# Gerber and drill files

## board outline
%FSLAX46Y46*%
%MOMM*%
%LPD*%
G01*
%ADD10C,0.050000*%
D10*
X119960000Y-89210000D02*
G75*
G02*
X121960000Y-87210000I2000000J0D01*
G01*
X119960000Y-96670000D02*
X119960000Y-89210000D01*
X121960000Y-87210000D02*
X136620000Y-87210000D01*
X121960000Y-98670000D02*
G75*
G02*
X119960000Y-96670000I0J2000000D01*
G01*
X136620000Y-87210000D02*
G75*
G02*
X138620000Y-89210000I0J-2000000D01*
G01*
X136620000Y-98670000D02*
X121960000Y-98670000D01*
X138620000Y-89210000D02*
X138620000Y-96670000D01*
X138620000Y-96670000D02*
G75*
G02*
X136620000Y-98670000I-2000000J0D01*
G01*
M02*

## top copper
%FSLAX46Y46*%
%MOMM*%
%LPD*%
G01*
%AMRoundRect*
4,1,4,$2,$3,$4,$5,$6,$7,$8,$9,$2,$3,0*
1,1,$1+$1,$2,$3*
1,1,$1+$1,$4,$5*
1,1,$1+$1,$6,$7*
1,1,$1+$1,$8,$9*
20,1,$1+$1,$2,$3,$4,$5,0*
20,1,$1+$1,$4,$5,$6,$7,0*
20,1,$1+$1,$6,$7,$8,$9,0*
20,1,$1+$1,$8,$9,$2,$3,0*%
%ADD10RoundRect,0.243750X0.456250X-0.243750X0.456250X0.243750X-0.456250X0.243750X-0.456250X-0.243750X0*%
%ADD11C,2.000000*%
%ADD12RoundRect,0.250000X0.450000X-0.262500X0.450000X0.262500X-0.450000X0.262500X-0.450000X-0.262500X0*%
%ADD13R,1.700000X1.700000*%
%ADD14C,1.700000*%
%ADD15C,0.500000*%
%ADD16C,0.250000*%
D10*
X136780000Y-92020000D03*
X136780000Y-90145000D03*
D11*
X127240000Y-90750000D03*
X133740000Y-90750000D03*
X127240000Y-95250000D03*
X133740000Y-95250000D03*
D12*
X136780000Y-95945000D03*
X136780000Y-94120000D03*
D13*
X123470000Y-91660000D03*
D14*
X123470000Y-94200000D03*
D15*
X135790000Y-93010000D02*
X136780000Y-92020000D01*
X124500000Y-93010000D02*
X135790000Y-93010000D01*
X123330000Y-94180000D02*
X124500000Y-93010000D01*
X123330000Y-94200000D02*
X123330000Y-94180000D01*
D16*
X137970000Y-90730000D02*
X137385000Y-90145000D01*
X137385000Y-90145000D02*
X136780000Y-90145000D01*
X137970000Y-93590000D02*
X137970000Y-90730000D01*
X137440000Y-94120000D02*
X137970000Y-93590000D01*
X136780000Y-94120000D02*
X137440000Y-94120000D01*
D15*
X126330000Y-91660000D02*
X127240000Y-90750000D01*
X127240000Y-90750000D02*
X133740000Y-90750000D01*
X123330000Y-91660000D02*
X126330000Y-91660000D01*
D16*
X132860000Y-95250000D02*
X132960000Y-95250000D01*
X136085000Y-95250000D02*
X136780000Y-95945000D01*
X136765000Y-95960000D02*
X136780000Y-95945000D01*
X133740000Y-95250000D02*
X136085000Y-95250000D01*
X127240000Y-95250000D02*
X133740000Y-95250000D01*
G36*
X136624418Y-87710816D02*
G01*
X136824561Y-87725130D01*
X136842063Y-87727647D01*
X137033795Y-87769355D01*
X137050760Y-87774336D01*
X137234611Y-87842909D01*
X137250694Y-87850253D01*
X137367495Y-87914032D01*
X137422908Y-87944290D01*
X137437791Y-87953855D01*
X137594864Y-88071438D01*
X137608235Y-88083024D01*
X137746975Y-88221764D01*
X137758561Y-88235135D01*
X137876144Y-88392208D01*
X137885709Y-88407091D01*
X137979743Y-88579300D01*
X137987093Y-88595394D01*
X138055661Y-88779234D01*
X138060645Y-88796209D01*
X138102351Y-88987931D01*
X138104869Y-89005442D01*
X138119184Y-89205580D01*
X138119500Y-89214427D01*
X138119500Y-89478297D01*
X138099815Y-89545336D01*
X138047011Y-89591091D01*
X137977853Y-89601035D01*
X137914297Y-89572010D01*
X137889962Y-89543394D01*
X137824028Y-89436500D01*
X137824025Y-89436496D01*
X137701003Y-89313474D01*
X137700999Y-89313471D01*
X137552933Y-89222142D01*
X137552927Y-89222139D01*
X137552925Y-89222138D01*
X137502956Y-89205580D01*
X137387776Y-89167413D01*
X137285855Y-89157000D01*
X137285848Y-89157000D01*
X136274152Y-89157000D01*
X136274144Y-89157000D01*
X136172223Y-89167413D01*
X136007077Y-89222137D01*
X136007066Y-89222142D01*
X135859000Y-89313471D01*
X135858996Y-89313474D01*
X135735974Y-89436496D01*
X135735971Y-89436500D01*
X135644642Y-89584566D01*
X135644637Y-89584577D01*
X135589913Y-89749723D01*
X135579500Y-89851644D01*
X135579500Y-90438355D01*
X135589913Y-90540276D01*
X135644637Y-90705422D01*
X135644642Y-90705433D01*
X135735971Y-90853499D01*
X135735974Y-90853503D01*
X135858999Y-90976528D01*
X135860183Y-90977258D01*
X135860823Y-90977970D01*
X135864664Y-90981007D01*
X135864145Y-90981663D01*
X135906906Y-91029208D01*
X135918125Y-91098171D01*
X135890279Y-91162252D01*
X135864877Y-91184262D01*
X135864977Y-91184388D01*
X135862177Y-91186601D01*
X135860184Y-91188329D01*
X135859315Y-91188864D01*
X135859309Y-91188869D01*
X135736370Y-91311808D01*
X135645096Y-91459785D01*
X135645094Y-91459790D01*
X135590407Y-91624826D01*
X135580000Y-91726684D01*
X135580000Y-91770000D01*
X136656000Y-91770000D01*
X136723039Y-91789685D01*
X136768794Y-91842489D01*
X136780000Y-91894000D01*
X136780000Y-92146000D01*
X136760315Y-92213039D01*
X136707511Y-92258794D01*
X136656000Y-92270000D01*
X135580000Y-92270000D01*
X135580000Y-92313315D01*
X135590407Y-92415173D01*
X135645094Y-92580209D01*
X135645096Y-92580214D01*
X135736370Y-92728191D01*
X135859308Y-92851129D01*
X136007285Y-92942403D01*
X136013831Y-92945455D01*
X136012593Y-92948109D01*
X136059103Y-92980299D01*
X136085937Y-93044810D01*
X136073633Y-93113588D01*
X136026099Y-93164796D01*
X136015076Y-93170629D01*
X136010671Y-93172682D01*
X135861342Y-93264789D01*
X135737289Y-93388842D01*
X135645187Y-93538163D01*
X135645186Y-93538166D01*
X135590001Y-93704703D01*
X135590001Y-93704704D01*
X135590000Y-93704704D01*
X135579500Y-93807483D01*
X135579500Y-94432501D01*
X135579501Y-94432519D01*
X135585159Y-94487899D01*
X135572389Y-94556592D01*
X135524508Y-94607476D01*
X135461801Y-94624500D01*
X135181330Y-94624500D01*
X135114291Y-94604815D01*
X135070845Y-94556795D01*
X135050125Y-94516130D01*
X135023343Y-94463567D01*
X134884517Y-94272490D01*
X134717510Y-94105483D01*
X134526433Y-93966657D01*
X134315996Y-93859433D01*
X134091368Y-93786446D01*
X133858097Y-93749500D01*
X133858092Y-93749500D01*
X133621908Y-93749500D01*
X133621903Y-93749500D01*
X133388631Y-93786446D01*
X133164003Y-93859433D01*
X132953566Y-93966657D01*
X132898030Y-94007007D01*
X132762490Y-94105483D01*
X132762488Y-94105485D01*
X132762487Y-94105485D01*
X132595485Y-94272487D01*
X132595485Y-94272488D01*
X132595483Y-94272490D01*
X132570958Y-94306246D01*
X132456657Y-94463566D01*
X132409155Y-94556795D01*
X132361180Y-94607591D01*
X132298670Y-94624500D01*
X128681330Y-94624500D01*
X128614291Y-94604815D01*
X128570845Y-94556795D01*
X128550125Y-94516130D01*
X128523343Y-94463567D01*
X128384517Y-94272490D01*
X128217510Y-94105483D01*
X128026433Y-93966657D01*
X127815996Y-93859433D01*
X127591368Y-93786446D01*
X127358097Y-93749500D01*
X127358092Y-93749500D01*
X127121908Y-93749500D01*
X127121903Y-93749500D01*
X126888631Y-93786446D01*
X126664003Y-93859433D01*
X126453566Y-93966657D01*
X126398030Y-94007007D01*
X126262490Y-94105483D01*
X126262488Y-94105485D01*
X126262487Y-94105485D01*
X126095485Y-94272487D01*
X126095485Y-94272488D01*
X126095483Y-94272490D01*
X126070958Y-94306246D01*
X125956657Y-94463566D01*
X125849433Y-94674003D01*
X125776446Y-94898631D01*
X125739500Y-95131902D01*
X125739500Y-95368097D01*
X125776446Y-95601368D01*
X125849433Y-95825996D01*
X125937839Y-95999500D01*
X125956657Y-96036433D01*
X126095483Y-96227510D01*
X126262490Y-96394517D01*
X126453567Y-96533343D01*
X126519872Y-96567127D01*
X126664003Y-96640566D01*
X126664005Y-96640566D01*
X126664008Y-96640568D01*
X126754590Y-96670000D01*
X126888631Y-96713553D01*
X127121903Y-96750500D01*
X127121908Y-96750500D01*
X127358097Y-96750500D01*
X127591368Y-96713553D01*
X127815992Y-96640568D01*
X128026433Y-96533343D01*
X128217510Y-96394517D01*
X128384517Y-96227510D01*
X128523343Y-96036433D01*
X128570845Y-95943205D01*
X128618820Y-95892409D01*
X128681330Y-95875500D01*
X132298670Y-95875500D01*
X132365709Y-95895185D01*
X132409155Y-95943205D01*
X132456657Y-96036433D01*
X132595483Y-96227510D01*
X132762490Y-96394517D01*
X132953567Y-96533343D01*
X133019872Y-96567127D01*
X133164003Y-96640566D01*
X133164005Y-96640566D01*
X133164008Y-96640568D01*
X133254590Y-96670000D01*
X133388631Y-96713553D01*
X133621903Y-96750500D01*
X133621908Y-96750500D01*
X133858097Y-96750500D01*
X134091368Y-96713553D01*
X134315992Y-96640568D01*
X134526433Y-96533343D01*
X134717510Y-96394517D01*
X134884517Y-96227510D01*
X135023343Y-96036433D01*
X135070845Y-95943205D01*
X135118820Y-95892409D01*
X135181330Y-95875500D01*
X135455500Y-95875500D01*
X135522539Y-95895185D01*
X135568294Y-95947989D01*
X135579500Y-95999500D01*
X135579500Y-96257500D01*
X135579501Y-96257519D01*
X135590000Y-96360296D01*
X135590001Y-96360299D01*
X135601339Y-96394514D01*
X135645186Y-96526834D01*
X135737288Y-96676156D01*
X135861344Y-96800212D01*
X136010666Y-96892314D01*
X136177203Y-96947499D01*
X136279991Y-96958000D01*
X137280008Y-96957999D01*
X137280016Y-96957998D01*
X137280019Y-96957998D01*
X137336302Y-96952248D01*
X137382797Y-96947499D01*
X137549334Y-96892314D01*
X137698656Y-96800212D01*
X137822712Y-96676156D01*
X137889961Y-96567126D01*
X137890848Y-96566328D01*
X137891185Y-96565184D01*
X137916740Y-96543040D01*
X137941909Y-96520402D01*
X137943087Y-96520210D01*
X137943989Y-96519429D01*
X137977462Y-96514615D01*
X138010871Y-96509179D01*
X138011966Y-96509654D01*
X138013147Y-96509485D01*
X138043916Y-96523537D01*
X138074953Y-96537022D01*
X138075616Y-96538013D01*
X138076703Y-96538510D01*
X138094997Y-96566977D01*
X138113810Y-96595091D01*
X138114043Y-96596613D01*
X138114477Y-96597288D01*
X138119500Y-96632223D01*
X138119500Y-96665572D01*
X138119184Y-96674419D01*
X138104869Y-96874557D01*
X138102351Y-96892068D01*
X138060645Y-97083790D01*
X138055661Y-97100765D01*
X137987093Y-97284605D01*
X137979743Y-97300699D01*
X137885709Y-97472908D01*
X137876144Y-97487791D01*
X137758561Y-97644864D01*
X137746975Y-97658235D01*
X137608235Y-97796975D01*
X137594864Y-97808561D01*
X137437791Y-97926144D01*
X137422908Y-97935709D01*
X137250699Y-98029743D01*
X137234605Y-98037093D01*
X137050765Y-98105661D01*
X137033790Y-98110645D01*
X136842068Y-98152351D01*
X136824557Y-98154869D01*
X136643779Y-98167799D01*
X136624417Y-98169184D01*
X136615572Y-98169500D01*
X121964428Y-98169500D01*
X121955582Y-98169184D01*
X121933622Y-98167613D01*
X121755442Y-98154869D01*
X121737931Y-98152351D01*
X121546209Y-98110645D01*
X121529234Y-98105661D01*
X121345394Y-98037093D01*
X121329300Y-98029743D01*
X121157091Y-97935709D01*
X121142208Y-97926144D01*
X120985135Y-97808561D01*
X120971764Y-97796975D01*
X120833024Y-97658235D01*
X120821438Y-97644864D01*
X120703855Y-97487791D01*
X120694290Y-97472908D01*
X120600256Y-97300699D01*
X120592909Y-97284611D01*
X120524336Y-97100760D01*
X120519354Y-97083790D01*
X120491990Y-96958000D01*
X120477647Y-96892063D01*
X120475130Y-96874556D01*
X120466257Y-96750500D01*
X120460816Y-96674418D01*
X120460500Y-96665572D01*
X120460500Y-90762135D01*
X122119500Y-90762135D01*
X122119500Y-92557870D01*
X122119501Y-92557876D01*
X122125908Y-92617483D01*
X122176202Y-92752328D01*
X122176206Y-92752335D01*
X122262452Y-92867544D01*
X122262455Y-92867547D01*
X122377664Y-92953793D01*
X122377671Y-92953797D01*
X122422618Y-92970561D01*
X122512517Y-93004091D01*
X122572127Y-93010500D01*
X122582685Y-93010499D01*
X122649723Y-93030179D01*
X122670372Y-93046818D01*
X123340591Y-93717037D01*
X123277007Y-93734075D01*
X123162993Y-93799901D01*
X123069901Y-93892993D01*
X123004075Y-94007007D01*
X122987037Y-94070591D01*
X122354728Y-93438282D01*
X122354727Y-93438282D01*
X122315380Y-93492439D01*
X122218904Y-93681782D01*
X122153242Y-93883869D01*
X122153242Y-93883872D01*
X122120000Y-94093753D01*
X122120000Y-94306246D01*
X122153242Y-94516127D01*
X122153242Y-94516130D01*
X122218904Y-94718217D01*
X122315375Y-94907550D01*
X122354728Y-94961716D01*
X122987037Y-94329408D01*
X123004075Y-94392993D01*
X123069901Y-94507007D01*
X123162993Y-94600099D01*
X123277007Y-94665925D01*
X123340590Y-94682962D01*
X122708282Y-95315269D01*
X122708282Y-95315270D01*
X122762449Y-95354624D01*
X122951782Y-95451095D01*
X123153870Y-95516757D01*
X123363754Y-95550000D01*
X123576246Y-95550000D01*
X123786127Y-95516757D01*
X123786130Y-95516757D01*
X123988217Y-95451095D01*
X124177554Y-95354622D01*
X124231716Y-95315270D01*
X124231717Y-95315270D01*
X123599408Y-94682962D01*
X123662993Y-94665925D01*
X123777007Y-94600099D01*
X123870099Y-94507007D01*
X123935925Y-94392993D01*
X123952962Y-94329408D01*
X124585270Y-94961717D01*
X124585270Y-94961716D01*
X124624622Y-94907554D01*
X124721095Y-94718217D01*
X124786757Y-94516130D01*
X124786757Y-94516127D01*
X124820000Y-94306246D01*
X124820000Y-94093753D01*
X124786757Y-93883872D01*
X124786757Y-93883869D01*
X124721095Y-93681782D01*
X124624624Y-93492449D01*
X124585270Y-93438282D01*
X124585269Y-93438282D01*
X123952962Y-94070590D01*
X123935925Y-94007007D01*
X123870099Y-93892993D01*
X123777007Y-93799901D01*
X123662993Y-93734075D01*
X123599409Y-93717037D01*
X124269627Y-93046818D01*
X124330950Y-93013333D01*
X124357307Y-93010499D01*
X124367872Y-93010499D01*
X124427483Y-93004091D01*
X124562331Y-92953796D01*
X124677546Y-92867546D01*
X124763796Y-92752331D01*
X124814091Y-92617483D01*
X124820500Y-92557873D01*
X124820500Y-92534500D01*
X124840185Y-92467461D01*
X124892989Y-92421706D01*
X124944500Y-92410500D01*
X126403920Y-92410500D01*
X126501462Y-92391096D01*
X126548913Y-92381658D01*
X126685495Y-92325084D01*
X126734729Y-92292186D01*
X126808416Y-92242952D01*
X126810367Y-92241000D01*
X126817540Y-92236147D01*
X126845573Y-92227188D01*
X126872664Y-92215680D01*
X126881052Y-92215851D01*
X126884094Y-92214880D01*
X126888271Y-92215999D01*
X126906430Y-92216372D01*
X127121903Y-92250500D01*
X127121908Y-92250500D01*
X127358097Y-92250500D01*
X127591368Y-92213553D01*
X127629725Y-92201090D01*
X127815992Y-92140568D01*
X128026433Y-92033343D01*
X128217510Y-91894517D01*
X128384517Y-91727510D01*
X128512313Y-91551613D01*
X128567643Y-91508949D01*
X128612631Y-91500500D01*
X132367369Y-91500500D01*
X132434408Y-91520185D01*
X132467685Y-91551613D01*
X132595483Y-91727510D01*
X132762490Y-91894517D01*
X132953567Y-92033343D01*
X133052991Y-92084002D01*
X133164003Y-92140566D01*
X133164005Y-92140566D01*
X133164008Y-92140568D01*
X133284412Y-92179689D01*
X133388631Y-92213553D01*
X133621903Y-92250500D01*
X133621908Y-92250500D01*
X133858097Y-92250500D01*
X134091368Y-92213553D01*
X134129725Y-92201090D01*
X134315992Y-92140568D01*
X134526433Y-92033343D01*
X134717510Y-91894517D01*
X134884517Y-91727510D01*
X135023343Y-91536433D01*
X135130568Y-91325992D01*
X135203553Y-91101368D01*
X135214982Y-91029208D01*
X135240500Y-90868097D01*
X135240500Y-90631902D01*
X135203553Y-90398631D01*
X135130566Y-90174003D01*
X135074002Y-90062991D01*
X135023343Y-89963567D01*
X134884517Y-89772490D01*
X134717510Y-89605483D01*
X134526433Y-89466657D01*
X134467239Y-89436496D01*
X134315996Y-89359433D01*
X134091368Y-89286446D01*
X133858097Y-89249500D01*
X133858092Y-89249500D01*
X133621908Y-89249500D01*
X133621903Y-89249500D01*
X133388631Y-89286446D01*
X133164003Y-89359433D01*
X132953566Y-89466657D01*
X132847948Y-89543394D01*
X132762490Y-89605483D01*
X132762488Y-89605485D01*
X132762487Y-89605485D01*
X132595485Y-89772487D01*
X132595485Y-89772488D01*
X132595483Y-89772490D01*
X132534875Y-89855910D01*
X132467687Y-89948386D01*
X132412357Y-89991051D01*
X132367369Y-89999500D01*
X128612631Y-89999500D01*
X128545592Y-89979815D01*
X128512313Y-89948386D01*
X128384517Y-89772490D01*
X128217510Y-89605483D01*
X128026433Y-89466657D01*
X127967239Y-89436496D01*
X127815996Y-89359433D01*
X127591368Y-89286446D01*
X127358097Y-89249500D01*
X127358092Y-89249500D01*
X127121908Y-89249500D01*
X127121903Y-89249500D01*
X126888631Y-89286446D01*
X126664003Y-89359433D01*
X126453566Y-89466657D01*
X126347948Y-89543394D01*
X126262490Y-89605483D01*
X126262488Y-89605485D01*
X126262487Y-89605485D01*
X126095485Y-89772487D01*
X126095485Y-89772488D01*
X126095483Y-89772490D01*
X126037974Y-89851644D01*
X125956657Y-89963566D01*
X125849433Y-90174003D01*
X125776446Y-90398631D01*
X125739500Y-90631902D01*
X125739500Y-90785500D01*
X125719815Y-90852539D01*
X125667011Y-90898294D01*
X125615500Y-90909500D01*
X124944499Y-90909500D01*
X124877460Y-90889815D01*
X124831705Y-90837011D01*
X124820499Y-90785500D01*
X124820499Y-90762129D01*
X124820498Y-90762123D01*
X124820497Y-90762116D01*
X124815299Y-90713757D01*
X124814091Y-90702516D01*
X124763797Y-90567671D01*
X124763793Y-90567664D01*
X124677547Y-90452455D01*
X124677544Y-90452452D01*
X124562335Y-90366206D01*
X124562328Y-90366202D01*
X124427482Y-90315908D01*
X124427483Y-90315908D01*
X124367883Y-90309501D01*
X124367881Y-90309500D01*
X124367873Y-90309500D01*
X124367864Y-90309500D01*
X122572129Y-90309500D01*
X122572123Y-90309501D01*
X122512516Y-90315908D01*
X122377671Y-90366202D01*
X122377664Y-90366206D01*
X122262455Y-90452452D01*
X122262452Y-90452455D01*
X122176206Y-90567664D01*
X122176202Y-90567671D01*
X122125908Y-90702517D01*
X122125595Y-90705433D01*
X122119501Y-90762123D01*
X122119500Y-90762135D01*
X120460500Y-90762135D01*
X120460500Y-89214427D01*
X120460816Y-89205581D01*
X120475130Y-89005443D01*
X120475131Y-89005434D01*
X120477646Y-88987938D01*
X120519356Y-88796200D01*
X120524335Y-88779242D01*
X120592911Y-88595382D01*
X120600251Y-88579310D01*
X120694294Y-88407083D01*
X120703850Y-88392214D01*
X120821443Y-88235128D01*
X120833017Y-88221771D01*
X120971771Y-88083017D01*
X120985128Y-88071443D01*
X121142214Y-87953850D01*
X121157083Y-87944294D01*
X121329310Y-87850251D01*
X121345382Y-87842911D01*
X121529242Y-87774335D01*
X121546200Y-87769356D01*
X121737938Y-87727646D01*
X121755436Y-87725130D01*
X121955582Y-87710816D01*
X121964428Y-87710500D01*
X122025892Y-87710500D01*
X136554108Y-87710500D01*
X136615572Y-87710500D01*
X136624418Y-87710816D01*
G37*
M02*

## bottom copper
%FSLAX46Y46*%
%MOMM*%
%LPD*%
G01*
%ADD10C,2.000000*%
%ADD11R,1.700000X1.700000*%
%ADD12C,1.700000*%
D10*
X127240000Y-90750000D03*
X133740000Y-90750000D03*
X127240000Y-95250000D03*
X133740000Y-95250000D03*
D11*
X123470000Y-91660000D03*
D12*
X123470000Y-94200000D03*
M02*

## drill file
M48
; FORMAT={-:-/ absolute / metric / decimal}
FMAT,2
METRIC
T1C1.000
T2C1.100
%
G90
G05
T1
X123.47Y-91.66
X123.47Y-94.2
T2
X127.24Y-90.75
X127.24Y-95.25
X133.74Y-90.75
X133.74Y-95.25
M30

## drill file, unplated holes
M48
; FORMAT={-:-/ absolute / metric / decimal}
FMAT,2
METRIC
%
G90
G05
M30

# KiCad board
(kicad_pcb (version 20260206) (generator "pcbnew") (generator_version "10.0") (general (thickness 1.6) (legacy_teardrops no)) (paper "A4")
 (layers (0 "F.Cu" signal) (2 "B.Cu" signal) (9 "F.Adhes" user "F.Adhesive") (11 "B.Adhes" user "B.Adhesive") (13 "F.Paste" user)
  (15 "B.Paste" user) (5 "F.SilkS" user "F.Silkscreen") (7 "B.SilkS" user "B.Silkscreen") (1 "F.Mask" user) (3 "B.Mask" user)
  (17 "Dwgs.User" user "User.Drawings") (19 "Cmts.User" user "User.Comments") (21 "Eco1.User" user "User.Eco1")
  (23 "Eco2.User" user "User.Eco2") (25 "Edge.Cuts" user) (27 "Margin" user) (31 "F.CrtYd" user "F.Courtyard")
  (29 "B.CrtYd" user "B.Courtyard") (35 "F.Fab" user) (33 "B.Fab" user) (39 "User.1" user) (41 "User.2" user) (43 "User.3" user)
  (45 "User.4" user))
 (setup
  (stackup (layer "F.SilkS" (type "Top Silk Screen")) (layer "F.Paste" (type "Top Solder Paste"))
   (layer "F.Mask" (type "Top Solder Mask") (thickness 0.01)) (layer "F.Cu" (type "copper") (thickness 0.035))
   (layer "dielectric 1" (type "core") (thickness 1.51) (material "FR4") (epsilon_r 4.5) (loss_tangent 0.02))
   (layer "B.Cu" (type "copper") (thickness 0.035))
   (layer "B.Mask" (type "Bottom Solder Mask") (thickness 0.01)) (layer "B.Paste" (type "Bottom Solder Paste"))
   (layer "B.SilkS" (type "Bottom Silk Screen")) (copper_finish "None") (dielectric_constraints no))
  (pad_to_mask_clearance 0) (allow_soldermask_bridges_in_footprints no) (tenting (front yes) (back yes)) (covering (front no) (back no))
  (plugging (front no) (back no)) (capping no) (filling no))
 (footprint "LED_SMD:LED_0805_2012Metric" (layer "F.Cu") (at 136.78 91.0825 90)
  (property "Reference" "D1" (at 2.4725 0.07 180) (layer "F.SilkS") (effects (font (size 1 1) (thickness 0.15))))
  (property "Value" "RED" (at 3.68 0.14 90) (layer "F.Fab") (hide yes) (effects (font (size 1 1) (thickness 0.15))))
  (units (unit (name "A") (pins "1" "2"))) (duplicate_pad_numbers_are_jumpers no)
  (pad "1" smd roundrect (at -0.9375 0 90) (size 0.975 1.4) (layers "F.Cu" "F.Mask" "F.Paste") (roundrect_rratio 0.25) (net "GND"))
  (pad "2" smd roundrect (at 0.9375 0 90) (size 0.975 1.4) (layers "F.Cu" "F.Mask" "F.Paste") (roundrect_rratio 0.25) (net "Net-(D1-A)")))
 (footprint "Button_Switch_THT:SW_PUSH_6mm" (layer "F.Cu") (at 127.24 90.75)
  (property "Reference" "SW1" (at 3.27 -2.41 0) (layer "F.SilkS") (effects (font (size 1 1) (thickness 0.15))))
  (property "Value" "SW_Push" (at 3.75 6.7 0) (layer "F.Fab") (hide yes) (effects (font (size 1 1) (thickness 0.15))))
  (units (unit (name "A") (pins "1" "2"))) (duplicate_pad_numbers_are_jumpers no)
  (pad "1" thru_hole circle (at 0 0 90) (size 2 2) (drill 1.1) (layers "*.Cu" "*.Mask") (remove_unused_layers no) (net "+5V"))
  (pad "1" thru_hole circle (at 6.5 0 90) (size 2 2) (drill 1.1) (layers "*.Cu" "*.Mask") (remove_unused_layers no) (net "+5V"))
  (pad "2" thru_hole circle (at 0 4.5 90) (size 2 2) (drill 1.1) (layers "*.Cu" "*.Mask") (remove_unused_layers no) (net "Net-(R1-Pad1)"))
  (pad "2" thru_hole circle (at 6.5 4.5 90) (size 2 2) (drill 1.1) (layers "*.Cu" "*.Mask") (remove_unused_layers no) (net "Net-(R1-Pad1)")))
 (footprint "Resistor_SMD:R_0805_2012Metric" (layer "F.Cu") (at 136.78 95.0325 90)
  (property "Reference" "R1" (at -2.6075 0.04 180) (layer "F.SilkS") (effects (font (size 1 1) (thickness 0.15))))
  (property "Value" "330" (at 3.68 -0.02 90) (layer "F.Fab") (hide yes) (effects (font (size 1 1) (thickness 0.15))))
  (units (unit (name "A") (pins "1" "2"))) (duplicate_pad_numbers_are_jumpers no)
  (pad "1" smd roundrect (at -0.9125 0 90) (size 1.025 1.4) (layers "F.Cu" "F.Mask" "F.Paste") (roundrect_rratio 0.243902)
   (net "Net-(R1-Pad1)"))
  (pad "2" smd roundrect (at 0.9125 0 90) (size 1.025 1.4) (layers "F.Cu" "F.Mask" "F.Paste") (roundrect_rratio 0.243902) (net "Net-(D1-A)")))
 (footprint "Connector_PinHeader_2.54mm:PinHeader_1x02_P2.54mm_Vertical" (layer "F.Cu") (at 123.47 91.66)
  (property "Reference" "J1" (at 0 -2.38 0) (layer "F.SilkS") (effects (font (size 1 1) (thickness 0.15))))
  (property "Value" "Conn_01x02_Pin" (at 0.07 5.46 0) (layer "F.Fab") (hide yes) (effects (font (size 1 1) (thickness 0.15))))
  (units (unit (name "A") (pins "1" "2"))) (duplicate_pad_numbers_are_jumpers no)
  (pad "1" thru_hole rect (at 0 0) (size 1.7 1.7) (drill 1) (layers "*.Cu" "*.Mask") (remove_unused_layers no) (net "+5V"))
  (pad "2" thru_hole circle (at 0 2.54) (size 1.7 1.7) (drill 1) (layers "*.Cu" "*.Mask") (remove_unused_layers no) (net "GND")))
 (gr_arc (start 119.96 89.21) (mid 120.545786 87.795786) (end 121.96 87.21) (stroke (width 0.05) (type default)) (layer "Edge.Cuts"))
 (gr_line (start 119.96 96.67) (end 119.96 89.21) (stroke (width 0.05) (type default)) (layer "Edge.Cuts"))
 (gr_line (start 121.96 87.21) (end 136.62 87.21) (stroke (width 0.05) (type default)) (layer "Edge.Cuts"))
 (gr_arc (start 121.96 98.67) (mid 120.545786 98.084214) (end 119.96 96.67) (stroke (width 0.05) (type default)) (layer "Edge.Cuts"))
 (gr_arc (start 136.62 87.21) (mid 138.034214 87.795786) (end 138.62 89.21) (stroke (width 0.05) (type default)) (layer "Edge.Cuts"))
 (gr_line (start 136.62 98.67) (end 121.96 98.67) (stroke (width 0.05) (type default)) (layer "Edge.Cuts"))
 (gr_line (start 138.62 89.21) (end 138.62 96.67) (stroke (width 0.05) (type default)) (layer "Edge.Cuts"))
 (gr_arc (start 138.62 96.67) (mid 138.034214 98.084214) (end 136.62 98.67) (stroke (width 0.05) (type default)) (layer "Edge.Cuts"))
 (segment (start 135.79 93.01) (end 136.78 92.02) (width 0.5) (layer "F.Cu") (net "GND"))
 (segment (start 124.5 93.01) (end 135.79 93.01) (width 0.5) (layer "F.Cu") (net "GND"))
 (segment (start 123.33 94.18) (end 124.5 93.01) (width 0.5) (layer "F.Cu") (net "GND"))
 (segment (start 123.33 94.2) (end 123.33 94.18) (width 0.5) (layer "F.Cu") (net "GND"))
 (segment (start 137.97 90.73) (end 137.385 90.145) (width 0.25) (layer "F.Cu") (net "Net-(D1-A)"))
 (segment (start 137.385 90.145) (end 136.78 90.145) (width 0.25) (layer "F.Cu") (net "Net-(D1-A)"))
 (segment (start 137.97 93.59) (end 137.97 90.73) (width 0.25) (layer "F.Cu") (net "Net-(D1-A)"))
 (segment (start 137.44 94.12) (end 137.97 93.59) (width 0.25) (layer "F.Cu") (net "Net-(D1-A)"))
 (segment (start 136.78 94.12) (end 137.44 94.12) (width 0.25) (layer "F.Cu") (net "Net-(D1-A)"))
 (segment (start 126.33 91.66) (end 127.24 90.75) (width 0.5) (layer "F.Cu") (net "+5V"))
 (segment (start 127.24 90.75) (end 133.74 90.75) (width 0.5) (layer "F.Cu") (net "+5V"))
 (segment (start 123.33 91.66) (end 126.33 91.66) (width 0.5) (layer "F.Cu") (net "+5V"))
 (segment (start 132.86 95.25) (end 132.96 95.25) (width 0.25) (layer "F.Cu") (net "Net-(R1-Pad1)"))
 (segment (start 136.085 95.25) (end 136.78 95.945) (width 0.25) (layer "F.Cu") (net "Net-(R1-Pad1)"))
 (segment (start 136.765 95.96) (end 136.78 95.945) (width 0.25) (layer "F.Cu") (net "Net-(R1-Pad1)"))
 (segment (start 133.74 95.25) (end 136.085 95.25) (width 0.25) (layer "F.Cu") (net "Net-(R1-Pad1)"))
 (segment (start 127.24 95.25) (end 133.74 95.25) (width 0.25) (layer "F.Cu") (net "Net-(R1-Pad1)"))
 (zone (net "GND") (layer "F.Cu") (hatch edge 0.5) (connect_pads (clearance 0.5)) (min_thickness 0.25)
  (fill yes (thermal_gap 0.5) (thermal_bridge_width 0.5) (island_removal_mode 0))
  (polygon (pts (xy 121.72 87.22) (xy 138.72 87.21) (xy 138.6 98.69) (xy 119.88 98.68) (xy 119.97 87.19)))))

